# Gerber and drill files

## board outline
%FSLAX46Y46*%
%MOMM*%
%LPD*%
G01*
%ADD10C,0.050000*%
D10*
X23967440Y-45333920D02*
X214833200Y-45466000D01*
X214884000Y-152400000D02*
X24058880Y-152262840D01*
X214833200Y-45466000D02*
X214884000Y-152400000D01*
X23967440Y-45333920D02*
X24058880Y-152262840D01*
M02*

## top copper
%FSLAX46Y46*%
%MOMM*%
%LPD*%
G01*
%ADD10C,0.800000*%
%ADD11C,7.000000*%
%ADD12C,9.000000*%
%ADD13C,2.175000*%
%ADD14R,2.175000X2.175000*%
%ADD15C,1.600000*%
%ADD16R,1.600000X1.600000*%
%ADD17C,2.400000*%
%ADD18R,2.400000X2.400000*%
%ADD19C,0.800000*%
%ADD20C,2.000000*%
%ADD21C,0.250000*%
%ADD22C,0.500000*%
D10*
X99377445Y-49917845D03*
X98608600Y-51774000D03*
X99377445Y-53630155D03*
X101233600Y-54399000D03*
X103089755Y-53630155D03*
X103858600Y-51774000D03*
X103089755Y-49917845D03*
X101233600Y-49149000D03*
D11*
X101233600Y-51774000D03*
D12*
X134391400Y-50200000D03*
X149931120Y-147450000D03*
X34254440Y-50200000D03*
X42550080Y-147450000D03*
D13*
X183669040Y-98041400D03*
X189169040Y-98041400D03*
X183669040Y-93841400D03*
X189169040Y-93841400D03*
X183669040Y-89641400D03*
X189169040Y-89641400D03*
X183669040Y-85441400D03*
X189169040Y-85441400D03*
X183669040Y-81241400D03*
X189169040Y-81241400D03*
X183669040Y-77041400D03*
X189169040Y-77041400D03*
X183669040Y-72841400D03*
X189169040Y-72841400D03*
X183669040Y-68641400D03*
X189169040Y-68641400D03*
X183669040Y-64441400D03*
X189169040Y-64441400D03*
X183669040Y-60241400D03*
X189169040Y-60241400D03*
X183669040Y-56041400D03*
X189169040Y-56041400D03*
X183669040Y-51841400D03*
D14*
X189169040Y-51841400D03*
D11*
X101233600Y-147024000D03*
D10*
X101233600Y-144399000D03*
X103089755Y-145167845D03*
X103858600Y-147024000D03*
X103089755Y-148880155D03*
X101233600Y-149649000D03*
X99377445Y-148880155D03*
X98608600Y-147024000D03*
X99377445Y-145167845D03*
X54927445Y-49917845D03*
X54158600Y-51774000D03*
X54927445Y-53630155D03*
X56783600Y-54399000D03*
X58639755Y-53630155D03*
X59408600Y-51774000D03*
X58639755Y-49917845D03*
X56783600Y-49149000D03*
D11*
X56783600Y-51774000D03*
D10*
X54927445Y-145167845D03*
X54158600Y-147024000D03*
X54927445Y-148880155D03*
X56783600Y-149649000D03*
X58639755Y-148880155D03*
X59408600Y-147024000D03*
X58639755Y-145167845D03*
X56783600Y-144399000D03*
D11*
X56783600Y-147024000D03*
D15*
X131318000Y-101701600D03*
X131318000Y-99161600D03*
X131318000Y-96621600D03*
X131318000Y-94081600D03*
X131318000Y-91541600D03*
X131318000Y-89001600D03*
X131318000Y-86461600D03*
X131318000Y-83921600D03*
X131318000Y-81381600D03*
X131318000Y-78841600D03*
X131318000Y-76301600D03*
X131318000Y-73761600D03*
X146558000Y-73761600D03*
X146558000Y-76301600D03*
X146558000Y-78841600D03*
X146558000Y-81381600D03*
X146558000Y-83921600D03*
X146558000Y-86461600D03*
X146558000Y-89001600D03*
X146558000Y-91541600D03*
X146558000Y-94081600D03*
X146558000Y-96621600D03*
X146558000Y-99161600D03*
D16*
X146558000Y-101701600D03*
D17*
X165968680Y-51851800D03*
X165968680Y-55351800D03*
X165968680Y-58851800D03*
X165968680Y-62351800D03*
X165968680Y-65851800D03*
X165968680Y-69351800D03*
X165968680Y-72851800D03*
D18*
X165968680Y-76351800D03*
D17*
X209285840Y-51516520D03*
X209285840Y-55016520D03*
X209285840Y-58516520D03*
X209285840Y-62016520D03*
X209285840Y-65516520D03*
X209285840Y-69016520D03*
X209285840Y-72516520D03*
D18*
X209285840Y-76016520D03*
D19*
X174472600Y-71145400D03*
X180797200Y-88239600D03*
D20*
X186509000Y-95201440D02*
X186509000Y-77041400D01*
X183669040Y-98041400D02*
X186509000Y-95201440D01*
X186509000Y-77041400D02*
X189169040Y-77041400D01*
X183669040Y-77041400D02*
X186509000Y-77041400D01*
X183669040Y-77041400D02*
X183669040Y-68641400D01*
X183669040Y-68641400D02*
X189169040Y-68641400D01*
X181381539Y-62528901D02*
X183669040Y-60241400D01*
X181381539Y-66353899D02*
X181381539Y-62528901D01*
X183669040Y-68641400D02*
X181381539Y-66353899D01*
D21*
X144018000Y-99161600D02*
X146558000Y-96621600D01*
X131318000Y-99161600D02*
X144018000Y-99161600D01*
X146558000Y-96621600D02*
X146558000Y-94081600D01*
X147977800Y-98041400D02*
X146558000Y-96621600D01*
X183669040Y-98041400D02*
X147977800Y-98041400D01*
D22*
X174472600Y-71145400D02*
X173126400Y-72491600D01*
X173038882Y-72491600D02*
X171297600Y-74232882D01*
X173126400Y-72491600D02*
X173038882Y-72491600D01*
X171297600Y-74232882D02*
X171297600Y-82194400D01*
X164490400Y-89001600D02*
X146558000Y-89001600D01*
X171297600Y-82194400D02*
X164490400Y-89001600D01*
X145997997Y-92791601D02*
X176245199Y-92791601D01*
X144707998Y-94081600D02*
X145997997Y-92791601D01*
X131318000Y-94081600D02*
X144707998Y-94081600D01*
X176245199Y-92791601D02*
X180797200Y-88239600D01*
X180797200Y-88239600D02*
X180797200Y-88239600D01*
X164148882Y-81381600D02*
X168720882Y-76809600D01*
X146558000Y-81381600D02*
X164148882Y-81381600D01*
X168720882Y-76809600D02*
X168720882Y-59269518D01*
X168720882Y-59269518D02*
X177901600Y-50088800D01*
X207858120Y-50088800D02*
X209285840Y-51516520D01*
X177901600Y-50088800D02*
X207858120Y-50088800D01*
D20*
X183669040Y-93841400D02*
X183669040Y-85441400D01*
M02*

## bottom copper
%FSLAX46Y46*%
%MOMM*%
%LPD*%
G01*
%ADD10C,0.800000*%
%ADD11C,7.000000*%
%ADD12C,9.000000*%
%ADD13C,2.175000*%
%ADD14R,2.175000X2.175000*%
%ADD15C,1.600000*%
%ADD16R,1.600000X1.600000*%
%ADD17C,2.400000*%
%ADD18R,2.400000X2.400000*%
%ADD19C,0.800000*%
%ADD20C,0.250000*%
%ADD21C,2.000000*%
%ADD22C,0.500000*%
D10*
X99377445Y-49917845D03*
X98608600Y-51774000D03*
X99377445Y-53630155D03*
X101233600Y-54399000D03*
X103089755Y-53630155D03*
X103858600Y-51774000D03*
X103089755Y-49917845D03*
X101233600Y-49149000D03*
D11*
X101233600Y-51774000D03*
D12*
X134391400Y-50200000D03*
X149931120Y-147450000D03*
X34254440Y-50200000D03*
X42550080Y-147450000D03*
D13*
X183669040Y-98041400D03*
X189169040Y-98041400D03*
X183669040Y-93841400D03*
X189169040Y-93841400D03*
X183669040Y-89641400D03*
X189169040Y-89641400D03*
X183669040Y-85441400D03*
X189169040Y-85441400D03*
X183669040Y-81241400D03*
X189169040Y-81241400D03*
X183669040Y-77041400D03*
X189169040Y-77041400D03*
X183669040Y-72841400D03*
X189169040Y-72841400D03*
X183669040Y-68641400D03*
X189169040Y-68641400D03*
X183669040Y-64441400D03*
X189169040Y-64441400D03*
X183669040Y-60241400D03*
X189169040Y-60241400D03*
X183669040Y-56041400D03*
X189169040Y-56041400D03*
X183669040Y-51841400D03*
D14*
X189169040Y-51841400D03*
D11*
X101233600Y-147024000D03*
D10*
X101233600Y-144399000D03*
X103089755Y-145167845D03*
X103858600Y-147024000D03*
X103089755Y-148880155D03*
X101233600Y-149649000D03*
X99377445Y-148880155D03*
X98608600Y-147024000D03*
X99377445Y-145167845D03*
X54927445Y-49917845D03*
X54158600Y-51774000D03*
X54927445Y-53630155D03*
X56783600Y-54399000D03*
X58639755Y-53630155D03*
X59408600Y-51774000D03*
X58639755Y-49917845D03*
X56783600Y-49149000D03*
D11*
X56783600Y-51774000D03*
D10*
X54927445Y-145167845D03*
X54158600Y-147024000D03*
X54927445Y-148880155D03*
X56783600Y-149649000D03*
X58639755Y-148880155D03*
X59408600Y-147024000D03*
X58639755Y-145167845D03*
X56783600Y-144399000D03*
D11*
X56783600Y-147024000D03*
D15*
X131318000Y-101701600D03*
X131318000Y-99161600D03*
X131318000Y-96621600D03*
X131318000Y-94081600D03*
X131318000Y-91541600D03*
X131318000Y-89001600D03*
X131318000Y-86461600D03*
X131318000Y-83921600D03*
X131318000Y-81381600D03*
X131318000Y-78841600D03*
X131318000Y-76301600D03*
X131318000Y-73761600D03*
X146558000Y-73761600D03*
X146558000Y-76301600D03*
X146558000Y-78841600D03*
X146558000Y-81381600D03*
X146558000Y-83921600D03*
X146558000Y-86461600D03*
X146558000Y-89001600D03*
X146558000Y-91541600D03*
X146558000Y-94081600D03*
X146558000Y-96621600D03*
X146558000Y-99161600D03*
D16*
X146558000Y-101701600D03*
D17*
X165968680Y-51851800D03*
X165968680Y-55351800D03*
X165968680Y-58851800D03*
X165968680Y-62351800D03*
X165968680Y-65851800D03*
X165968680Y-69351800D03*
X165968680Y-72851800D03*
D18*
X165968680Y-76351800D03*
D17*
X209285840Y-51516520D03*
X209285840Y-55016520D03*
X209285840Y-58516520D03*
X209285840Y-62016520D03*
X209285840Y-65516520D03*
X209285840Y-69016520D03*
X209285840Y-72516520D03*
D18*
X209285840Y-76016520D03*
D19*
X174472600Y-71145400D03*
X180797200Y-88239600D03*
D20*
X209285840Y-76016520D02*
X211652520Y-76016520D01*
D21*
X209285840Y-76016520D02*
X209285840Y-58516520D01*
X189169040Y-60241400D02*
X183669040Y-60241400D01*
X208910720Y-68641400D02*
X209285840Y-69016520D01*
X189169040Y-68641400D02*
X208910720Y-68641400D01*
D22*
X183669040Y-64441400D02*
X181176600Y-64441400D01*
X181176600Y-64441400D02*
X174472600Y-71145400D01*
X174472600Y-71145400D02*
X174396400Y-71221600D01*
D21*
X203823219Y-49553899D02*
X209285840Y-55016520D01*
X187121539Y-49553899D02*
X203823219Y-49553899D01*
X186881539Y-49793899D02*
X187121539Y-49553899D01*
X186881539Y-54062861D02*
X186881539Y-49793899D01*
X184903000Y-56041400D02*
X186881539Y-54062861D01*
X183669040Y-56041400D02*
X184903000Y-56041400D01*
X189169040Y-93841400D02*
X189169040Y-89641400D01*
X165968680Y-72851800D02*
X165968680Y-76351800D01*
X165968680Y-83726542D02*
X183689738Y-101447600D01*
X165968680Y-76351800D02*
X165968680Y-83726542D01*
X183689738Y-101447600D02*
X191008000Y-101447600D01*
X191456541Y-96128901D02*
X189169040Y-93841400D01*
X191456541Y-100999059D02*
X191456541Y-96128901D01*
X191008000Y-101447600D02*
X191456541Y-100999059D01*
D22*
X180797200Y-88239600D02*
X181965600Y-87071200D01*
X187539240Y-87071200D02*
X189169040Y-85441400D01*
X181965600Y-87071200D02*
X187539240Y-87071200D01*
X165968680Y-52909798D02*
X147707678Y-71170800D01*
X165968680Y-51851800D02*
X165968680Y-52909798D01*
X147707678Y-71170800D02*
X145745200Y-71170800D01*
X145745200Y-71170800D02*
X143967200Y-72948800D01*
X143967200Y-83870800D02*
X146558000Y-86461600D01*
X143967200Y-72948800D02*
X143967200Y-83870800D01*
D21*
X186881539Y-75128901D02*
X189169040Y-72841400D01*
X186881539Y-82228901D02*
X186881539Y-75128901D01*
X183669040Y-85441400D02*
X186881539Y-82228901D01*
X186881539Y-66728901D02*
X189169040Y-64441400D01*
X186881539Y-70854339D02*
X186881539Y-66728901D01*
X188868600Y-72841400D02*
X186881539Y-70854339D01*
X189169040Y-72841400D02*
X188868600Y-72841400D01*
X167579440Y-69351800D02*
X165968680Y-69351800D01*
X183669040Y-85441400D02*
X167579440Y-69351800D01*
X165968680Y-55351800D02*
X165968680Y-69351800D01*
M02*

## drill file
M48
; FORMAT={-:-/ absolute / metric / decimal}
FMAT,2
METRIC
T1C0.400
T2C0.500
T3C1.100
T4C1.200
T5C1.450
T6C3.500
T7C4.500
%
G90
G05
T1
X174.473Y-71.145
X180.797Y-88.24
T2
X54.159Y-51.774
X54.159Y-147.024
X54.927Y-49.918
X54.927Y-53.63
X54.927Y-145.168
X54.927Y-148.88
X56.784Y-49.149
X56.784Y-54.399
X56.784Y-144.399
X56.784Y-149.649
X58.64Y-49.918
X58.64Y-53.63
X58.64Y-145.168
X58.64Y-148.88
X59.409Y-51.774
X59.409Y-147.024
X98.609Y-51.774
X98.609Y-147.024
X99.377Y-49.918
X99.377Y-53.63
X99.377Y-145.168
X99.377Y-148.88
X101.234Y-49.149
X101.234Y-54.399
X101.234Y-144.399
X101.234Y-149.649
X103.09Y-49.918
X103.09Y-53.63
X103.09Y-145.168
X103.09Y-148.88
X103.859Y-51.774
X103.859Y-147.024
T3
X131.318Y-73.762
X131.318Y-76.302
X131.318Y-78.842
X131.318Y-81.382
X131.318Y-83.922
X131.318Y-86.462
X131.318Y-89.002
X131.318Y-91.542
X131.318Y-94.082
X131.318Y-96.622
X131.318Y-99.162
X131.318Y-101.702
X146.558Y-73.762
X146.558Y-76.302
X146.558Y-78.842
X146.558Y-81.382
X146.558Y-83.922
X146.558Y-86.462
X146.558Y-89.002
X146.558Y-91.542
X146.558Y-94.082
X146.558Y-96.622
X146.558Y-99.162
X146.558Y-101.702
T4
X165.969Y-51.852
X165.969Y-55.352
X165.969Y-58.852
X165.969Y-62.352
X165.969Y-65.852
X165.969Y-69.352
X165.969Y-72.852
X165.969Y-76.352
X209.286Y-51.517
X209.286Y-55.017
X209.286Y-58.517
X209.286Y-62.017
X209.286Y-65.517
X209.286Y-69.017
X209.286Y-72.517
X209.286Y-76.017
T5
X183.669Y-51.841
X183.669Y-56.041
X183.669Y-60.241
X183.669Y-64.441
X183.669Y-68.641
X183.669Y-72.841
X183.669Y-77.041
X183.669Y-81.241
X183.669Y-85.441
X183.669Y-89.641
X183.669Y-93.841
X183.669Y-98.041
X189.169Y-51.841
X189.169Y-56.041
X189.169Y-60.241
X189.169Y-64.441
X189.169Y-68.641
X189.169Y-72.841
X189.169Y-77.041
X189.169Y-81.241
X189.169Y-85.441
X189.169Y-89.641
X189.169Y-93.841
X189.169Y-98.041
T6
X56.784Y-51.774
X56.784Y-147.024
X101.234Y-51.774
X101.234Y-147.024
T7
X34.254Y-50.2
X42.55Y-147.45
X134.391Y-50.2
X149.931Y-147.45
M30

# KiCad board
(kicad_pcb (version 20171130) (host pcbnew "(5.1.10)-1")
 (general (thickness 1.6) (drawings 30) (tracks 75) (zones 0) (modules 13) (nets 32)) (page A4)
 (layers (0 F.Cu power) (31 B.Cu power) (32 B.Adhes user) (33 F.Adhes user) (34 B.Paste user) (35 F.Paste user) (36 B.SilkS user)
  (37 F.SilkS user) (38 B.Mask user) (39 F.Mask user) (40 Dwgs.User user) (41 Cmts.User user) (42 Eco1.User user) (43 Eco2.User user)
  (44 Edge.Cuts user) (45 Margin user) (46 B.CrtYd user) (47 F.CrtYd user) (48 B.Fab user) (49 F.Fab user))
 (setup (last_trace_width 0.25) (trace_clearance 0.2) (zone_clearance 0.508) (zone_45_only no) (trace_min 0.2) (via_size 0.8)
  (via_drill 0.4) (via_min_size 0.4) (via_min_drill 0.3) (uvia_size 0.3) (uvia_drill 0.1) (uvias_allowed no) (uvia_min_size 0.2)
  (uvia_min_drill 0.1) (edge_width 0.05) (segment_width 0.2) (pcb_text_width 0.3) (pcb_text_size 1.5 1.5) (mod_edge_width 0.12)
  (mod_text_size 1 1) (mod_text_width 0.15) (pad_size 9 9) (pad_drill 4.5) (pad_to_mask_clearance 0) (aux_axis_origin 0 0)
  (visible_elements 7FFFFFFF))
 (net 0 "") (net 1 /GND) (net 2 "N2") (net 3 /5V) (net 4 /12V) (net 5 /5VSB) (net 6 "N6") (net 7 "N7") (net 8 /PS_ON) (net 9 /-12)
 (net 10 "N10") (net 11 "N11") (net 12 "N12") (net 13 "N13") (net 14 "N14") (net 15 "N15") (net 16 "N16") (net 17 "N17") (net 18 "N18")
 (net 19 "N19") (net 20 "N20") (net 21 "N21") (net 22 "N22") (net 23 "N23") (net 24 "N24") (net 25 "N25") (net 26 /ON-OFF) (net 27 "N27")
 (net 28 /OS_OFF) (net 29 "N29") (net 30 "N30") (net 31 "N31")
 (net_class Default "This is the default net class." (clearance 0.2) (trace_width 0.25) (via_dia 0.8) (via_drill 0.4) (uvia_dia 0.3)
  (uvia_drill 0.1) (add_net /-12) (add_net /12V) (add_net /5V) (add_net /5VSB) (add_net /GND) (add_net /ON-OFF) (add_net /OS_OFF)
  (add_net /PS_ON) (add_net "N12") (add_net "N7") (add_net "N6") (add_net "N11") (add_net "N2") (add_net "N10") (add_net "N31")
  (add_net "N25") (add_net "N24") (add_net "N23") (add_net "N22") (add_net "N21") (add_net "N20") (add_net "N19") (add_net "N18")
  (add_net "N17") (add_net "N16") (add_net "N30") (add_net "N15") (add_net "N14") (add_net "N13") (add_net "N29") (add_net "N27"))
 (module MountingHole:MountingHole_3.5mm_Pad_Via (layer F.Cu) (at 101.2336 51.774 90)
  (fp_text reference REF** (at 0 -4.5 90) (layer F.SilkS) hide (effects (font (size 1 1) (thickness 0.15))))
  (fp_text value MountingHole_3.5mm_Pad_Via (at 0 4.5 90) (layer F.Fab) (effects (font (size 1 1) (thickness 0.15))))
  (pad 1 thru_hole circle (at 1.856155 -1.856155 90) (size 0.8 0.8) (drill 0.5) (layers *.Cu *.Mask))
  (pad 1 thru_hole circle (at 0 -2.625 90) (size 0.8 0.8) (drill 0.5) (layers *.Cu *.Mask))
  (pad 1 thru_hole circle (at -1.856155 -1.856155 90) (size 0.8 0.8) (drill 0.5) (layers *.Cu *.Mask))
  (pad 1 thru_hole circle (at -2.625 0 90) (size 0.8 0.8) (drill 0.5) (layers *.Cu *.Mask))
  (pad 1 thru_hole circle (at -1.856155 1.856155 90) (size 0.8 0.8) (drill 0.5) (layers *.Cu *.Mask))
  (pad 1 thru_hole circle (at 0 2.625 90) (size 0.8 0.8) (drill 0.5) (layers *.Cu *.Mask))
  (pad 1 thru_hole circle (at 1.856155 1.856155 90) (size 0.8 0.8) (drill 0.5) (layers *.Cu *.Mask))
  (pad 1 thru_hole circle (at 2.625 0 90) (size 0.8 0.8) (drill 0.5) (layers *.Cu *.Mask))
  (pad 1 thru_hole circle (at 0 0 90) (size 7 7) (drill 3.5) (layers *.Mask F.Cu)))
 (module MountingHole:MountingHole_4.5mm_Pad (layer F.Cu) (at 134.3914 50.2)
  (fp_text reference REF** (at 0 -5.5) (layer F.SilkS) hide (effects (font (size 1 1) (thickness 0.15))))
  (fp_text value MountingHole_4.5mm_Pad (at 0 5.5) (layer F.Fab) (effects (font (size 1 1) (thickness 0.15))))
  (pad 1 thru_hole circle (at 0 0) (size 9 9) (drill 4.5) (layers *.Mask F.Cu)))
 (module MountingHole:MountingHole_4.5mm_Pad (layer F.Cu) (at 149.93112 147.45)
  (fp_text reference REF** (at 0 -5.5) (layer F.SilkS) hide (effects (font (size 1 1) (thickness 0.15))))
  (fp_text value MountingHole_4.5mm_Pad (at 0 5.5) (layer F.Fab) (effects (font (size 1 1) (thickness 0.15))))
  (pad 1 thru_hole circle (at 0 0) (size 9 9) (drill 4.5) (layers *.Mask F.Cu)))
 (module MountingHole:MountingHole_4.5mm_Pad (layer F.Cu) (at 34.25444 50.2)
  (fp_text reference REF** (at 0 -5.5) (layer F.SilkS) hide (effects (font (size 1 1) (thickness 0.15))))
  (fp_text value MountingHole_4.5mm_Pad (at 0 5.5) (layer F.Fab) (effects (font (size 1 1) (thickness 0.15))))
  (pad 1 thru_hole circle (at 0 0) (size 9 9) (drill 4.5) (layers *.Mask F.Cu)))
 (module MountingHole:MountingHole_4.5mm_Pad (layer F.Cu) (at 42.55008 147.45)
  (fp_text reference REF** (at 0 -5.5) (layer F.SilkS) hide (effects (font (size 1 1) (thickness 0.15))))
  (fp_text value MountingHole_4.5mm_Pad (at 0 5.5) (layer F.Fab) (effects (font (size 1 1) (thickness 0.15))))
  (pad 1 thru_hole circle (at 0 0) (size 9 9) (drill 4.5) (layers *.Mask F.Cu)))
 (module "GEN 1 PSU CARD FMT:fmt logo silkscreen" (layer B.Cu) (at 80.4164 89.0524 180)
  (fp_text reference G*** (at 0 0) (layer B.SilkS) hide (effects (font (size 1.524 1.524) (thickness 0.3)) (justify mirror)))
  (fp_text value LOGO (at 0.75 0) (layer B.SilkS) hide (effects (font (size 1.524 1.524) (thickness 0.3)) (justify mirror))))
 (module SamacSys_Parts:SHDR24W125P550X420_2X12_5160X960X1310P (layer F.Cu) (at 189.16904 51.8414 270)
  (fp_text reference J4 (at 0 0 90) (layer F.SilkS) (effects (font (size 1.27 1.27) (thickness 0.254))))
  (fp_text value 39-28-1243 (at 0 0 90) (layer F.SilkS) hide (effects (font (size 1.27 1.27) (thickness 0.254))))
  (pad 24 thru_hole circle (at 46.2 5.5) (size 2.175 2.175) (drill 1.45) (layers *.Cu *.Mask F.SilkS) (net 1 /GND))
  (pad 23 thru_hole circle (at 46.2 0) (size 2.175 2.175) (drill 1.45) (layers *.Cu *.Mask F.SilkS) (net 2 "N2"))
  (pad 22 thru_hole circle (at 42 5.5) (size 2.175 2.175) (drill 1.45) (layers *.Cu *.Mask F.SilkS) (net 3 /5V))
  (pad 21 thru_hole circle (at 42 0) (size 2.175 2.175) (drill 1.45) (layers *.Cu *.Mask F.SilkS) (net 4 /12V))
  (pad 20 thru_hole circle (at 37.8 5.5) (size 2.175 2.175) (drill 1.45) (layers *.Cu *.Mask F.SilkS) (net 3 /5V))
  (pad 19 thru_hole circle (at 37.8 0) (size 2.175 2.175) (drill 1.45) (layers *.Cu *.Mask F.SilkS) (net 4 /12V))
  (pad 18 thru_hole circle (at 33.6 5.5) (size 2.175 2.175) (drill 1.45) (layers *.Cu *.Mask F.SilkS) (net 3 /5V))
  (pad 17 thru_hole circle (at 33.6 0) (size 2.175 2.175) (drill 1.45) (layers *.Cu *.Mask F.SilkS) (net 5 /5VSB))
  (pad 16 thru_hole circle (at 29.4 5.5) (size 2.175 2.175) (drill 1.45) (layers *.Cu *.Mask F.SilkS) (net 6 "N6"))
  (pad 15 thru_hole circle (at 29.4 0) (size 2.175 2.175) (drill 1.45) (layers *.Cu *.Mask F.SilkS) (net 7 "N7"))
  (pad 14 thru_hole circle (at 25.2 5.5) (size 2.175 2.175) (drill 1.45) (layers *.Cu *.Mask F.SilkS) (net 1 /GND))
  (pad 13 thru_hole circle (at 25.2 0) (size 2.175 2.175) (drill 1.45) (layers *.Cu *.Mask F.SilkS) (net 1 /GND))
  (pad 12 thru_hole circle (at 21 5.5) (size 2.175 2.175) (drill 1.45) (layers *.Cu *.Mask F.SilkS) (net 1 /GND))
  (pad 11 thru_hole circle (at 21 0) (size 2.175 2.175) (drill 1.45) (layers *.Cu *.Mask F.SilkS) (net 3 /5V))
  (pad 10 thru_hole circle (at 16.8 5.5) (size 2.175 2.175) (drill 1.45) (layers *.Cu *.Mask F.SilkS) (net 1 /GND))
  (pad 9 thru_hole circle (at 16.8 0) (size 2.175 2.175) (drill 1.45) (layers *.Cu *.Mask F.SilkS) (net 1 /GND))
  (pad 8 thru_hole circle (at 12.6 5.5) (size 2.175 2.175) (drill 1.45) (layers *.Cu *.Mask F.SilkS) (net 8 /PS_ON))
  (pad 7 thru_hole circle (at 12.6 0) (size 2.175 2.175) (drill 1.45) (layers *.Cu *.Mask F.SilkS) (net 3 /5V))
  (pad 6 thru_hole circle (at 8.4 5.5) (size 2.175 2.175) (drill 1.45) (layers *.Cu *.Mask F.SilkS) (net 1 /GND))
  (pad 5 thru_hole circle (at 8.4 0) (size 2.175 2.175) (drill 1.45) (layers *.Cu *.Mask F.SilkS) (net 1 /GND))
  (pad 4 thru_hole circle (at 4.2 5.5) (size 2.175 2.175) (drill 1.45) (layers *.Cu *.Mask F.SilkS) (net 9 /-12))
  (pad 3 thru_hole circle (at 4.2 0) (size 2.175 2.175) (drill 1.45) (layers *.Cu *.Mask F.SilkS) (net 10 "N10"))
  (pad 2 thru_hole circle (at 0 5.5) (size 2.175 2.175) (drill 1.45) (layers *.Cu *.Mask F.SilkS) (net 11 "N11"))
  (pad 1 thru_hole rect (at 0 0) (size 2.175 2.175) (drill 1.45) (layers *.Cu *.Mask F.SilkS) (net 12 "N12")))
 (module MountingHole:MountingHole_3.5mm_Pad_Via (layer F.Cu) (at 101.2336 147.024 90)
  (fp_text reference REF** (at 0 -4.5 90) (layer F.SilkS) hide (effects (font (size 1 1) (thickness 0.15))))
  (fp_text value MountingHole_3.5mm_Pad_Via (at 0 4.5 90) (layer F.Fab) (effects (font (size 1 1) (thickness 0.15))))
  (pad 1 thru_hole circle (at 0 0 90) (size 7 7) (drill 3.5) (layers *.Mask F.Cu))
  (pad 1 thru_hole circle (at 2.625 0 90) (size 0.8 0.8) (drill 0.5) (layers *.Cu *.Mask))
  (pad 1 thru_hole circle (at 1.856155 1.856155 90) (size 0.8 0.8) (drill 0.5) (layers *.Cu *.Mask))
  (pad 1 thru_hole circle (at 0 2.625 90) (size 0.8 0.8) (drill 0.5) (layers *.Cu *.Mask))
  (pad 1 thru_hole circle (at -1.856155 1.856155 90) (size 0.8 0.8) (drill 0.5) (layers *.Cu *.Mask))
  (pad 1 thru_hole circle (at -2.625 0 90) (size 0.8 0.8) (drill 0.5) (layers *.Cu *.Mask))
  (pad 1 thru_hole circle (at -1.856155 -1.856155 90) (size 0.8 0.8) (drill 0.5) (layers *.Cu *.Mask))
  (pad 1 thru_hole circle (at 0 -2.625 90) (size 0.8 0.8) (drill 0.5) (layers *.Cu *.Mask))
  (pad 1 thru_hole circle (at 1.856155 -1.856155 90) (size 0.8 0.8) (drill 0.5) (layers *.Cu *.Mask)))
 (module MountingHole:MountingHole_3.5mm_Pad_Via (layer F.Cu) (at 56.7836 51.774 90)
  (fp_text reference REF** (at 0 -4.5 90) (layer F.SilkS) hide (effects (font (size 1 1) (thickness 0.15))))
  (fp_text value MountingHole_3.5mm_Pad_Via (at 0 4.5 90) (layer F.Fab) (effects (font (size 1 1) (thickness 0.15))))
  (pad 1 thru_hole circle (at 1.856155 -1.856155 90) (size 0.8 0.8) (drill 0.5) (layers *.Cu *.Mask))
  (pad 1 thru_hole circle (at 0 -2.625 90) (size 0.8 0.8) (drill 0.5) (layers *.Cu *.Mask))
  (pad 1 thru_hole circle (at -1.856155 -1.856155 90) (size 0.8 0.8) (drill 0.5) (layers *.Cu *.Mask))
  (pad 1 thru_hole circle (at -2.625 0 90) (size 0.8 0.8) (drill 0.5) (layers *.Cu *.Mask))
  (pad 1 thru_hole circle (at -1.856155 1.856155 90) (size 0.8 0.8) (drill 0.5) (layers *.Cu *.Mask))
  (pad 1 thru_hole circle (at 0 2.625 90) (size 0.8 0.8) (drill 0.5) (layers *.Cu *.Mask))
  (pad 1 thru_hole circle (at 1.856155 1.856155 90) (size 0.8 0.8) (drill 0.5) (layers *.Cu *.Mask))
  (pad 1 thru_hole circle (at 2.625 0 90) (size 0.8 0.8) (drill 0.5) (layers *.Cu *.Mask))
  (pad 1 thru_hole circle (at 0 0 90) (size 7 7) (drill 3.5) (layers *.Mask F.Cu)))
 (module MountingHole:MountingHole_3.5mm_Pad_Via (layer F.Cu) (at 56.7836 147.024 90)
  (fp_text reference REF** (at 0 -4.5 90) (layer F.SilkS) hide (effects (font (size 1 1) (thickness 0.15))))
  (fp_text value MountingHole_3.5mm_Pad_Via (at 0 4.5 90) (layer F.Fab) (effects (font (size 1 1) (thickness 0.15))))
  (pad 1 thru_hole circle (at 1.856155 -1.856155 90) (size 0.8 0.8) (drill 0.5) (layers *.Cu *.Mask))
  (pad 1 thru_hole circle (at 0 -2.625 90) (size 0.8 0.8) (drill 0.5) (layers *.Cu *.Mask))
  (pad 1 thru_hole circle (at -1.856155 -1.856155 90) (size 0.8 0.8) (drill 0.5) (layers *.Cu *.Mask))
  (pad 1 thru_hole circle (at -2.625 0 90) (size 0.8 0.8) (drill 0.5) (layers *.Cu *.Mask))
  (pad 1 thru_hole circle (at -1.856155 1.856155 90) (size 0.8 0.8) (drill 0.5) (layers *.Cu *.Mask))
  (pad 1 thru_hole circle (at 0 2.625 90) (size 0.8 0.8) (drill 0.5) (layers *.Cu *.Mask))
  (pad 1 thru_hole circle (at 1.856155 1.856155 90) (size 0.8 0.8) (drill 0.5) (layers *.Cu *.Mask))
  (pad 1 thru_hole circle (at 2.625 0 90) (size 0.8 0.8) (drill 0.5) (layers *.Cu *.Mask))
  (pad 1 thru_hole circle (at 0 0 90) (size 7 7) (drill 3.5) (layers *.Mask F.Cu)))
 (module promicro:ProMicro (layer F.Cu) (at 138.938 87.7316 90)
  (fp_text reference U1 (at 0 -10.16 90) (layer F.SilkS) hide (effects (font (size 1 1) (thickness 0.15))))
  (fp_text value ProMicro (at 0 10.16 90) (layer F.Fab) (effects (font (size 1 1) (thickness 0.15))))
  (pad 24 thru_hole circle (at -13.97 -7.62 90) (size 1.6 1.6) (drill 1.1) (layers *.Cu *.Mask F.SilkS) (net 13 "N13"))
  (pad 23 thru_hole circle (at -11.43 -7.62 90) (size 1.6 1.6) (drill 1.1) (layers *.Cu *.Mask F.SilkS) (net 1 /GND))
  (pad 22 thru_hole circle (at -8.89 -7.62 90) (size 1.6 1.6) (drill 1.1) (layers *.Cu *.Mask F.SilkS) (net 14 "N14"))
  (pad 21 thru_hole circle (at -6.35 -7.62 90) (size 1.6 1.6) (drill 1.1) (layers *.Cu *.Mask F.SilkS) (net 5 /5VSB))
  (pad 20 thru_hole circle (at -3.81 -7.62 90) (size 1.6 1.6) (drill 1.1) (layers *.Cu *.Mask F.SilkS) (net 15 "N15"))
  (pad 19 thru_hole circle (at -1.27 -7.62 90) (size 1.6 1.6) (drill 1.1) (layers *.Cu *.Mask F.SilkS) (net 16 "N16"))
  (pad 18 thru_hole circle (at 1.27 -7.62 90) (size 1.6 1.6) (drill 1.1) (layers *.Cu *.Mask F.SilkS) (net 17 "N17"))
  (pad 17 thru_hole circle (at 3.81 -7.62 90) (size 1.6 1.6) (drill 1.1) (layers *.Cu *.Mask F.SilkS) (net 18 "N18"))
  (pad 16 thru_hole circle (at 6.35 -7.62 90) (size 1.6 1.6) (drill 1.1) (layers *.Cu *.Mask F.SilkS) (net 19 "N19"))
  (pad 15 thru_hole circle (at 8.89 -7.62 90) (size 1.6 1.6) (drill 1.1) (layers *.Cu *.Mask F.SilkS) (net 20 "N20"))
  (pad 14 thru_hole circle (at 11.43 -7.62 90) (size 1.6 1.6) (drill 1.1) (layers *.Cu *.Mask F.SilkS) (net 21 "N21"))
  (pad 13 thru_hole circle (at 13.97 -7.62 90) (size 1.6 1.6) (drill 1.1) (layers *.Cu *.Mask F.SilkS) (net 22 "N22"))
  (pad 12 thru_hole circle (at 13.97 7.62 90) (size 1.6 1.6) (drill 1.1) (layers *.Cu *.Mask F.SilkS) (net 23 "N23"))
  (pad 11 thru_hole circle (at 11.43 7.62 90) (size 1.6 1.6) (drill 1.1) (layers *.Cu *.Mask F.SilkS) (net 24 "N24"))
  (pad 10 thru_hole circle (at 8.89 7.62 90) (size 1.6 1.6) (drill 1.1) (layers *.Cu *.Mask F.SilkS) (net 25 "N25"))
  (pad 9 thru_hole circle (at 6.35 7.62 90) (size 1.6 1.6) (drill 1.1) (layers *.Cu *.Mask F.SilkS) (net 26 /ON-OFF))
  (pad 8 thru_hole circle (at 3.81 7.62 90) (size 1.6 1.6) (drill 1.1) (layers *.Cu *.Mask F.SilkS) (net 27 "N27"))
  (pad 7 thru_hole circle (at 1.27 7.62 90) (size 1.6 1.6) (drill 1.1) (layers *.Cu *.Mask F.SilkS) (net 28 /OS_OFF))
  (pad 6 thru_hole circle (at -1.27 7.62 90) (size 1.6 1.6) (drill 1.1) (layers *.Cu *.Mask F.SilkS) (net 8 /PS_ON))
  (pad 5 thru_hole circle (at -3.81 7.62 90) (size 1.6 1.6) (drill 1.1) (layers *.Cu *.Mask F.SilkS) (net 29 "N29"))
  (pad 4 thru_hole circle (at -6.35 7.62 90) (size 1.6 1.6) (drill 1.1) (layers *.Cu *.Mask F.SilkS) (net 1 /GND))
  (pad 3 thru_hole circle (at -8.89 7.62 90) (size 1.6 1.6) (drill 1.1) (layers *.Cu *.Mask F.SilkS) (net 1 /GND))
  (pad 2 thru_hole circle (at -11.43 7.62 90) (size 1.6 1.6) (drill 1.1) (layers *.Cu *.Mask F.SilkS) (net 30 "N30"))
  (pad 1 thru_hole rect (at -13.97 7.62 90) (size 1.6 1.6) (drill 1.1) (layers *.Cu *.Mask F.SilkS) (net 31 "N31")))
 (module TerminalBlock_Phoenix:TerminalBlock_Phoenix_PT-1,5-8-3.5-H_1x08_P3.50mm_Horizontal (layer F.Cu) (at 165.96868 76.3518 90)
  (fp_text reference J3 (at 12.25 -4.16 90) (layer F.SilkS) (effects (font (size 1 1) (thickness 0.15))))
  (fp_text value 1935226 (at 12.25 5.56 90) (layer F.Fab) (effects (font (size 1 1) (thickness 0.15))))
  (pad 8 thru_hole circle (at 24.5 0 90) (size 2.4 2.4) (drill 1.2) (layers *.Cu *.Mask) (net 28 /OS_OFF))
  (pad 7 thru_hole circle (at 21 0 90) (size 2.4 2.4) (drill 1.2) (layers *.Cu *.Mask) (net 3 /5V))
  (pad 6 thru_hole circle (at 17.5 0 90) (size 2.4 2.4) (drill 1.2) (layers *.Cu *.Mask) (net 3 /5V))
  (pad 5 thru_hole circle (at 14 0 90) (size 2.4 2.4) (drill 1.2) (layers *.Cu *.Mask) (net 3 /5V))
  (pad 4 thru_hole circle (at 10.5 0 90) (size 2.4 2.4) (drill 1.2) (layers *.Cu *.Mask) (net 3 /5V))
  (pad 3 thru_hole circle (at 7 0 90) (size 2.4 2.4) (drill 1.2) (layers *.Cu *.Mask) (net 3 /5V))
  (pad 2 thru_hole circle (at 3.5 0 90) (size 2.4 2.4) (drill 1.2) (layers *.Cu *.Mask) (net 4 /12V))
  (pad 1 thru_hole rect (at 0 0 90) (size 2.4 2.4) (drill 1.2) (layers *.Cu *.Mask) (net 4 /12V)))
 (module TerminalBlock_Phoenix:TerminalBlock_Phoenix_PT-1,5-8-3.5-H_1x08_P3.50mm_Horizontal (layer F.Cu) (at 209.28584 76.01652 90)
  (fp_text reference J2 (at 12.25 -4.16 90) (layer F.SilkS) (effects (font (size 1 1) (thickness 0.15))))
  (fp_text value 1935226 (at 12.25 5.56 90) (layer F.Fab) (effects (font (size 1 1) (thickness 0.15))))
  (pad 8 thru_hole circle (at 24.5 0 90) (size 2.4 2.4) (drill 1.2) (layers *.Cu *.Mask) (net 26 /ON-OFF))
  (pad 7 thru_hole circle (at 21 0 90) (size 2.4 2.4) (drill 1.2) (layers *.Cu *.Mask) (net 9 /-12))
  (pad 6 thru_hole circle (at 17.5 0 90) (size 2.4 2.4) (drill 1.2) (layers *.Cu *.Mask) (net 1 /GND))
  (pad 5 thru_hole circle (at 14 0 90) (size 2.4 2.4) (drill 1.2) (layers *.Cu *.Mask) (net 1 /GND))
  (pad 4 thru_hole circle (at 10.5 0 90) (size 2.4 2.4) (drill 1.2) (layers *.Cu *.Mask) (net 1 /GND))
  (pad 3 thru_hole circle (at 7 0 90) (size 2.4 2.4) (drill 1.2) (layers *.Cu *.Mask) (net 1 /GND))
  (pad 2 thru_hole circle (at 3.5 0 90) (size 2.4 2.4) (drill 1.2) (layers *.Cu *.Mask) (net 1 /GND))
  (pad 1 thru_hole rect (at 0 0 90) (size 2.4 2.4) (drill 1.2) (layers *.Cu *.Mask) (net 1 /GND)))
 (gr_line (start 23.96744 45.33392) (end 214.8332 45.466) (layer Edge.Cuts) (width 0.05))
 (gr_line (start 214.884 152.4) (end 24.05888 152.26284) (layer Edge.Cuts) (width 0.05))
 (gr_line (start 214.8332 45.466) (end 214.884 152.4) (layer Edge.Cuts) (width 0.05))
 (gr_line (start 23.96744 45.33392) (end 24.05888 152.26284) (layer Edge.Cuts) (width 0.05))
 (segment (start 209.28584 76.01652) (end 211.65252 76.01652) (width 0.25) (layer B.Cu) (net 1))
 (segment (start 209.28584 76.01652) (end 209.28584 58.51652) (width 2) (layer B.Cu) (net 1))
 (segment (start 189.16904 60.2414) (end 183.66904 60.2414) (width 2) (layer B.Cu) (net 1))
 (segment (start 186.509 95.20144) (end 186.509 77.0414) (width 2) (layer F.Cu) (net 1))
 (segment (start 183.66904 98.0414) (end 186.509 95.20144) (width 2) (layer F.Cu) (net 1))
 (segment (start 186.509 77.0414) (end 189.16904 77.0414) (width 2) (layer F.Cu) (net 1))
 (segment (start 183.66904 77.0414) (end 186.509 77.0414) (width 2) (layer F.Cu) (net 1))
 (segment (start 183.66904 77.0414) (end 183.66904 68.6414) (width 2) (layer F.Cu) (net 1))
 (segment (start 183.66904 68.6414) (end 189.16904 68.6414) (width 2) (layer F.Cu) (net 1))
 (segment (start 181.381539 62.528901) (end 183.66904 60.2414) (width 2) (layer F.Cu) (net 1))
 (segment (start 181.381539 66.353899) (end 181.381539 62.528901) (width 2) (layer F.Cu) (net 1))
 (segment (start 183.66904 68.6414) (end 181.381539 66.353899) (width 2) (layer F.Cu) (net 1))
 (segment (start 208.91072 68.6414) (end 209.28584 69.01652) (width 2) (layer B.Cu) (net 1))
 (segment (start 189.16904 68.6414) (end 208.91072 68.6414) (width 2) (layer B.Cu) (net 1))
 (segment (start 144.018 99.1616) (end 146.558 96.6216) (width 0.25) (layer F.Cu) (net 1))
 (segment (start 131.318 99.1616) (end 144.018 99.1616) (width 0.25) (layer F.Cu) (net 1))
 (segment (start 146.558 96.6216) (end 146.558 94.0816) (width 0.25) (layer F.Cu) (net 1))
 (segment (start 147.9778 98.0414) (end 146.558 96.6216) (width 0.25) (layer F.Cu) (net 1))
 (segment (start 183.66904 98.0414) (end 147.9778 98.0414) (width 0.25) (layer F.Cu) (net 1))
 (segment (start 183.66904 64.4414) (end 181.1766 64.4414) (width 0.5) (layer B.Cu) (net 8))
 (segment (start 181.1766 64.4414) (end 174.4726 71.1454) (width 0.5) (layer B.Cu) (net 8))
 (segment (start 174.4726 71.1454) (end 174.3964 71.2216) (width 0.5) (layer B.Cu) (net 8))
 (via (at 174.4726 71.1454) (size 0.8) (drill 0.4) (layers F.Cu B.Cu) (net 8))
 (segment (start 174.4726 71.1454) (end 173.1264 72.4916) (width 0.5) (layer F.Cu) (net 8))
 (segment (start 173.038882 72.4916) (end 171.2976 74.232882) (width 0.5) (layer F.Cu) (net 8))
 (segment (start 173.1264 72.4916) (end 173.038882 72.4916) (width 0.5) (layer F.Cu) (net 8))
 (segment (start 171.2976 74.232882) (end 171.2976 82.1944) (width 0.5) (layer F.Cu) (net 8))
 (segment (start 164.4904 89.0016) (end 146.558 89.0016) (width 0.5) (layer F.Cu) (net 8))
 (segment (start 171.2976 82.1944) (end 164.4904 89.0016) (width 0.5) (layer F.Cu) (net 8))
 (segment (start 203.823219 49.553899) (end 209.28584 55.01652) (width 2) (layer B.Cu) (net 9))
 (segment (start 187.121539 49.553899) (end 203.823219 49.553899) (width 2) (layer B.Cu) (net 9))
 (segment (start 186.881539 49.793899) (end 187.121539 49.553899) (width 2) (layer B.Cu) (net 9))
 (segment (start 186.881539 54.062861) (end 186.881539 49.793899) (width 2) (layer B.Cu) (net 9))
 (segment (start 184.903 56.0414) (end 186.881539 54.062861) (width 2) (layer B.Cu) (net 9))
 (segment (start 183.66904 56.0414) (end 184.903 56.0414) (width 2) (layer B.Cu) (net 9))
 (segment (start 189.16904 93.8414) (end 189.16904 89.6414) (width 2) (layer B.Cu) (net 4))
 (segment (start 165.96868 72.8518) (end 165.96868 76.3518) (width 2) (layer B.Cu) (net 4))
 (segment (start 165.96868 83.726542) (end 183.689738 101.4476) (width 2) (layer B.Cu) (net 4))
 (segment (start 165.96868 76.3518) (end 165.96868 83.726542) (width 2) (layer B.Cu) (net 4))
 (segment (start 183.689738 101.4476) (end 191.008 101.4476) (width 2) (layer B.Cu) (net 4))
 (segment (start 191.456541 96.128901) (end 189.16904 93.8414) (width 2) (layer B.Cu) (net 4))
 (segment (start 191.456541 100.999059) (end 191.456541 96.128901) (width 2) (layer B.Cu) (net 4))
 (segment (start 191.008 101.4476) (end 191.456541 100.999059) (width 2) (layer B.Cu) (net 4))
 (segment (start 145.997997 92.791601) (end 176.245199 92.791601) (width 0.5) (layer F.Cu) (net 5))
 (segment (start 144.707998 94.0816) (end 145.997997 92.791601) (width 0.5) (layer F.Cu) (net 5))
 (segment (start 131.318 94.0816) (end 144.707998 94.0816) (width 0.5) (layer F.Cu) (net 5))
 (segment (start 176.245199 92.791601) (end 180.7972 88.2396) (width 0.5) (layer F.Cu) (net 5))
 (segment (start 180.7972 88.2396) (end 180.7972 88.2396) (width 0.5) (layer F.Cu) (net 5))
 (via (at 180.7972 88.2396) (size 0.8) (drill 0.4) (layers F.Cu B.Cu) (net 5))
 (segment (start 180.7972 88.2396) (end 181.9656 87.0712) (width 0.5) (layer B.Cu) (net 5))
 (segment (start 187.53924 87.0712) (end 189.16904 85.4414) (width 0.5) (layer B.Cu) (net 5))
 (segment (start 181.9656 87.0712) (end 187.53924 87.0712) (width 0.5) (layer B.Cu) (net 5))
 (segment (start 164.148882 81.3816) (end 168.720882 76.8096) (width 0.5) (layer F.Cu) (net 26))
 (segment (start 146.558 81.3816) (end 164.148882 81.3816) (width 0.5) (layer F.Cu) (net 26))
 (segment (start 168.720882 76.8096) (end 168.720882 59.269518) (width 0.5) (layer F.Cu) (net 26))
 (segment (start 168.720882 59.269518) (end 177.9016 50.0888) (width 0.5) (layer F.Cu) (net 26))
 (segment (start 207.85812 50.0888) (end 209.28584 51.51652) (width 0.5) (layer F.Cu) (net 26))
 (segment (start 177.9016 50.0888) (end 207.85812 50.0888) (width 0.5) (layer F.Cu) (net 26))
 (segment (start 165.96868 52.909798) (end 147.707678 71.1708) (width 0.5) (layer B.Cu) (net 28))
 (segment (start 165.96868 51.8518) (end 165.96868 52.909798) (width 0.5) (layer B.Cu) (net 28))
 (segment (start 147.707678 71.1708) (end 145.7452 71.1708) (width 0.5) (layer B.Cu) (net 28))
 (segment (start 145.7452 71.1708) (end 143.9672 72.9488) (width 0.5) (layer B.Cu) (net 28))
 (segment (start 143.9672 83.8708) (end 146.558 86.4616) (width 0.5) (layer B.Cu) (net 28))
 (segment (start 143.9672 72.9488) (end 143.9672 83.8708) (width 0.5) (layer B.Cu) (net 28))
 (segment (start 183.66904 93.8414) (end 183.66904 85.4414) (width 2) (layer F.Cu) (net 3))
 (segment (start 186.881539 75.128901) (end 189.16904 72.8414) (width 2) (layer B.Cu) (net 3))
 (segment (start 186.881539 82.228901) (end 186.881539 75.128901) (width 2) (layer B.Cu) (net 3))
 (segment (start 183.66904 85.4414) (end 186.881539 82.228901) (width 2) (layer B.Cu) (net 3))
 (segment (start 186.881539 66.728901) (end 189.16904 64.4414) (width 2) (layer B.Cu) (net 3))
 (segment (start 186.881539 70.854339) (end 186.881539 66.728901) (width 2) (layer B.Cu) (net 3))
 (segment (start 188.8686 72.8414) (end 186.881539 70.854339) (width 2) (layer B.Cu) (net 3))
 (segment (start 189.16904 72.8414) (end 188.8686 72.8414) (width 2) (layer B.Cu) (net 3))
 (segment (start 167.57944 69.3518) (end 165.96868 69.3518) (width 2) (layer B.Cu) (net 3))
 (segment (start 183.66904 85.4414) (end 167.57944 69.3518) (width 2) (layer B.Cu) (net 3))
 (segment (start 165.96868 55.3518) (end 165.96868 69.3518) (width 2) (layer B.Cu) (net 3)))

